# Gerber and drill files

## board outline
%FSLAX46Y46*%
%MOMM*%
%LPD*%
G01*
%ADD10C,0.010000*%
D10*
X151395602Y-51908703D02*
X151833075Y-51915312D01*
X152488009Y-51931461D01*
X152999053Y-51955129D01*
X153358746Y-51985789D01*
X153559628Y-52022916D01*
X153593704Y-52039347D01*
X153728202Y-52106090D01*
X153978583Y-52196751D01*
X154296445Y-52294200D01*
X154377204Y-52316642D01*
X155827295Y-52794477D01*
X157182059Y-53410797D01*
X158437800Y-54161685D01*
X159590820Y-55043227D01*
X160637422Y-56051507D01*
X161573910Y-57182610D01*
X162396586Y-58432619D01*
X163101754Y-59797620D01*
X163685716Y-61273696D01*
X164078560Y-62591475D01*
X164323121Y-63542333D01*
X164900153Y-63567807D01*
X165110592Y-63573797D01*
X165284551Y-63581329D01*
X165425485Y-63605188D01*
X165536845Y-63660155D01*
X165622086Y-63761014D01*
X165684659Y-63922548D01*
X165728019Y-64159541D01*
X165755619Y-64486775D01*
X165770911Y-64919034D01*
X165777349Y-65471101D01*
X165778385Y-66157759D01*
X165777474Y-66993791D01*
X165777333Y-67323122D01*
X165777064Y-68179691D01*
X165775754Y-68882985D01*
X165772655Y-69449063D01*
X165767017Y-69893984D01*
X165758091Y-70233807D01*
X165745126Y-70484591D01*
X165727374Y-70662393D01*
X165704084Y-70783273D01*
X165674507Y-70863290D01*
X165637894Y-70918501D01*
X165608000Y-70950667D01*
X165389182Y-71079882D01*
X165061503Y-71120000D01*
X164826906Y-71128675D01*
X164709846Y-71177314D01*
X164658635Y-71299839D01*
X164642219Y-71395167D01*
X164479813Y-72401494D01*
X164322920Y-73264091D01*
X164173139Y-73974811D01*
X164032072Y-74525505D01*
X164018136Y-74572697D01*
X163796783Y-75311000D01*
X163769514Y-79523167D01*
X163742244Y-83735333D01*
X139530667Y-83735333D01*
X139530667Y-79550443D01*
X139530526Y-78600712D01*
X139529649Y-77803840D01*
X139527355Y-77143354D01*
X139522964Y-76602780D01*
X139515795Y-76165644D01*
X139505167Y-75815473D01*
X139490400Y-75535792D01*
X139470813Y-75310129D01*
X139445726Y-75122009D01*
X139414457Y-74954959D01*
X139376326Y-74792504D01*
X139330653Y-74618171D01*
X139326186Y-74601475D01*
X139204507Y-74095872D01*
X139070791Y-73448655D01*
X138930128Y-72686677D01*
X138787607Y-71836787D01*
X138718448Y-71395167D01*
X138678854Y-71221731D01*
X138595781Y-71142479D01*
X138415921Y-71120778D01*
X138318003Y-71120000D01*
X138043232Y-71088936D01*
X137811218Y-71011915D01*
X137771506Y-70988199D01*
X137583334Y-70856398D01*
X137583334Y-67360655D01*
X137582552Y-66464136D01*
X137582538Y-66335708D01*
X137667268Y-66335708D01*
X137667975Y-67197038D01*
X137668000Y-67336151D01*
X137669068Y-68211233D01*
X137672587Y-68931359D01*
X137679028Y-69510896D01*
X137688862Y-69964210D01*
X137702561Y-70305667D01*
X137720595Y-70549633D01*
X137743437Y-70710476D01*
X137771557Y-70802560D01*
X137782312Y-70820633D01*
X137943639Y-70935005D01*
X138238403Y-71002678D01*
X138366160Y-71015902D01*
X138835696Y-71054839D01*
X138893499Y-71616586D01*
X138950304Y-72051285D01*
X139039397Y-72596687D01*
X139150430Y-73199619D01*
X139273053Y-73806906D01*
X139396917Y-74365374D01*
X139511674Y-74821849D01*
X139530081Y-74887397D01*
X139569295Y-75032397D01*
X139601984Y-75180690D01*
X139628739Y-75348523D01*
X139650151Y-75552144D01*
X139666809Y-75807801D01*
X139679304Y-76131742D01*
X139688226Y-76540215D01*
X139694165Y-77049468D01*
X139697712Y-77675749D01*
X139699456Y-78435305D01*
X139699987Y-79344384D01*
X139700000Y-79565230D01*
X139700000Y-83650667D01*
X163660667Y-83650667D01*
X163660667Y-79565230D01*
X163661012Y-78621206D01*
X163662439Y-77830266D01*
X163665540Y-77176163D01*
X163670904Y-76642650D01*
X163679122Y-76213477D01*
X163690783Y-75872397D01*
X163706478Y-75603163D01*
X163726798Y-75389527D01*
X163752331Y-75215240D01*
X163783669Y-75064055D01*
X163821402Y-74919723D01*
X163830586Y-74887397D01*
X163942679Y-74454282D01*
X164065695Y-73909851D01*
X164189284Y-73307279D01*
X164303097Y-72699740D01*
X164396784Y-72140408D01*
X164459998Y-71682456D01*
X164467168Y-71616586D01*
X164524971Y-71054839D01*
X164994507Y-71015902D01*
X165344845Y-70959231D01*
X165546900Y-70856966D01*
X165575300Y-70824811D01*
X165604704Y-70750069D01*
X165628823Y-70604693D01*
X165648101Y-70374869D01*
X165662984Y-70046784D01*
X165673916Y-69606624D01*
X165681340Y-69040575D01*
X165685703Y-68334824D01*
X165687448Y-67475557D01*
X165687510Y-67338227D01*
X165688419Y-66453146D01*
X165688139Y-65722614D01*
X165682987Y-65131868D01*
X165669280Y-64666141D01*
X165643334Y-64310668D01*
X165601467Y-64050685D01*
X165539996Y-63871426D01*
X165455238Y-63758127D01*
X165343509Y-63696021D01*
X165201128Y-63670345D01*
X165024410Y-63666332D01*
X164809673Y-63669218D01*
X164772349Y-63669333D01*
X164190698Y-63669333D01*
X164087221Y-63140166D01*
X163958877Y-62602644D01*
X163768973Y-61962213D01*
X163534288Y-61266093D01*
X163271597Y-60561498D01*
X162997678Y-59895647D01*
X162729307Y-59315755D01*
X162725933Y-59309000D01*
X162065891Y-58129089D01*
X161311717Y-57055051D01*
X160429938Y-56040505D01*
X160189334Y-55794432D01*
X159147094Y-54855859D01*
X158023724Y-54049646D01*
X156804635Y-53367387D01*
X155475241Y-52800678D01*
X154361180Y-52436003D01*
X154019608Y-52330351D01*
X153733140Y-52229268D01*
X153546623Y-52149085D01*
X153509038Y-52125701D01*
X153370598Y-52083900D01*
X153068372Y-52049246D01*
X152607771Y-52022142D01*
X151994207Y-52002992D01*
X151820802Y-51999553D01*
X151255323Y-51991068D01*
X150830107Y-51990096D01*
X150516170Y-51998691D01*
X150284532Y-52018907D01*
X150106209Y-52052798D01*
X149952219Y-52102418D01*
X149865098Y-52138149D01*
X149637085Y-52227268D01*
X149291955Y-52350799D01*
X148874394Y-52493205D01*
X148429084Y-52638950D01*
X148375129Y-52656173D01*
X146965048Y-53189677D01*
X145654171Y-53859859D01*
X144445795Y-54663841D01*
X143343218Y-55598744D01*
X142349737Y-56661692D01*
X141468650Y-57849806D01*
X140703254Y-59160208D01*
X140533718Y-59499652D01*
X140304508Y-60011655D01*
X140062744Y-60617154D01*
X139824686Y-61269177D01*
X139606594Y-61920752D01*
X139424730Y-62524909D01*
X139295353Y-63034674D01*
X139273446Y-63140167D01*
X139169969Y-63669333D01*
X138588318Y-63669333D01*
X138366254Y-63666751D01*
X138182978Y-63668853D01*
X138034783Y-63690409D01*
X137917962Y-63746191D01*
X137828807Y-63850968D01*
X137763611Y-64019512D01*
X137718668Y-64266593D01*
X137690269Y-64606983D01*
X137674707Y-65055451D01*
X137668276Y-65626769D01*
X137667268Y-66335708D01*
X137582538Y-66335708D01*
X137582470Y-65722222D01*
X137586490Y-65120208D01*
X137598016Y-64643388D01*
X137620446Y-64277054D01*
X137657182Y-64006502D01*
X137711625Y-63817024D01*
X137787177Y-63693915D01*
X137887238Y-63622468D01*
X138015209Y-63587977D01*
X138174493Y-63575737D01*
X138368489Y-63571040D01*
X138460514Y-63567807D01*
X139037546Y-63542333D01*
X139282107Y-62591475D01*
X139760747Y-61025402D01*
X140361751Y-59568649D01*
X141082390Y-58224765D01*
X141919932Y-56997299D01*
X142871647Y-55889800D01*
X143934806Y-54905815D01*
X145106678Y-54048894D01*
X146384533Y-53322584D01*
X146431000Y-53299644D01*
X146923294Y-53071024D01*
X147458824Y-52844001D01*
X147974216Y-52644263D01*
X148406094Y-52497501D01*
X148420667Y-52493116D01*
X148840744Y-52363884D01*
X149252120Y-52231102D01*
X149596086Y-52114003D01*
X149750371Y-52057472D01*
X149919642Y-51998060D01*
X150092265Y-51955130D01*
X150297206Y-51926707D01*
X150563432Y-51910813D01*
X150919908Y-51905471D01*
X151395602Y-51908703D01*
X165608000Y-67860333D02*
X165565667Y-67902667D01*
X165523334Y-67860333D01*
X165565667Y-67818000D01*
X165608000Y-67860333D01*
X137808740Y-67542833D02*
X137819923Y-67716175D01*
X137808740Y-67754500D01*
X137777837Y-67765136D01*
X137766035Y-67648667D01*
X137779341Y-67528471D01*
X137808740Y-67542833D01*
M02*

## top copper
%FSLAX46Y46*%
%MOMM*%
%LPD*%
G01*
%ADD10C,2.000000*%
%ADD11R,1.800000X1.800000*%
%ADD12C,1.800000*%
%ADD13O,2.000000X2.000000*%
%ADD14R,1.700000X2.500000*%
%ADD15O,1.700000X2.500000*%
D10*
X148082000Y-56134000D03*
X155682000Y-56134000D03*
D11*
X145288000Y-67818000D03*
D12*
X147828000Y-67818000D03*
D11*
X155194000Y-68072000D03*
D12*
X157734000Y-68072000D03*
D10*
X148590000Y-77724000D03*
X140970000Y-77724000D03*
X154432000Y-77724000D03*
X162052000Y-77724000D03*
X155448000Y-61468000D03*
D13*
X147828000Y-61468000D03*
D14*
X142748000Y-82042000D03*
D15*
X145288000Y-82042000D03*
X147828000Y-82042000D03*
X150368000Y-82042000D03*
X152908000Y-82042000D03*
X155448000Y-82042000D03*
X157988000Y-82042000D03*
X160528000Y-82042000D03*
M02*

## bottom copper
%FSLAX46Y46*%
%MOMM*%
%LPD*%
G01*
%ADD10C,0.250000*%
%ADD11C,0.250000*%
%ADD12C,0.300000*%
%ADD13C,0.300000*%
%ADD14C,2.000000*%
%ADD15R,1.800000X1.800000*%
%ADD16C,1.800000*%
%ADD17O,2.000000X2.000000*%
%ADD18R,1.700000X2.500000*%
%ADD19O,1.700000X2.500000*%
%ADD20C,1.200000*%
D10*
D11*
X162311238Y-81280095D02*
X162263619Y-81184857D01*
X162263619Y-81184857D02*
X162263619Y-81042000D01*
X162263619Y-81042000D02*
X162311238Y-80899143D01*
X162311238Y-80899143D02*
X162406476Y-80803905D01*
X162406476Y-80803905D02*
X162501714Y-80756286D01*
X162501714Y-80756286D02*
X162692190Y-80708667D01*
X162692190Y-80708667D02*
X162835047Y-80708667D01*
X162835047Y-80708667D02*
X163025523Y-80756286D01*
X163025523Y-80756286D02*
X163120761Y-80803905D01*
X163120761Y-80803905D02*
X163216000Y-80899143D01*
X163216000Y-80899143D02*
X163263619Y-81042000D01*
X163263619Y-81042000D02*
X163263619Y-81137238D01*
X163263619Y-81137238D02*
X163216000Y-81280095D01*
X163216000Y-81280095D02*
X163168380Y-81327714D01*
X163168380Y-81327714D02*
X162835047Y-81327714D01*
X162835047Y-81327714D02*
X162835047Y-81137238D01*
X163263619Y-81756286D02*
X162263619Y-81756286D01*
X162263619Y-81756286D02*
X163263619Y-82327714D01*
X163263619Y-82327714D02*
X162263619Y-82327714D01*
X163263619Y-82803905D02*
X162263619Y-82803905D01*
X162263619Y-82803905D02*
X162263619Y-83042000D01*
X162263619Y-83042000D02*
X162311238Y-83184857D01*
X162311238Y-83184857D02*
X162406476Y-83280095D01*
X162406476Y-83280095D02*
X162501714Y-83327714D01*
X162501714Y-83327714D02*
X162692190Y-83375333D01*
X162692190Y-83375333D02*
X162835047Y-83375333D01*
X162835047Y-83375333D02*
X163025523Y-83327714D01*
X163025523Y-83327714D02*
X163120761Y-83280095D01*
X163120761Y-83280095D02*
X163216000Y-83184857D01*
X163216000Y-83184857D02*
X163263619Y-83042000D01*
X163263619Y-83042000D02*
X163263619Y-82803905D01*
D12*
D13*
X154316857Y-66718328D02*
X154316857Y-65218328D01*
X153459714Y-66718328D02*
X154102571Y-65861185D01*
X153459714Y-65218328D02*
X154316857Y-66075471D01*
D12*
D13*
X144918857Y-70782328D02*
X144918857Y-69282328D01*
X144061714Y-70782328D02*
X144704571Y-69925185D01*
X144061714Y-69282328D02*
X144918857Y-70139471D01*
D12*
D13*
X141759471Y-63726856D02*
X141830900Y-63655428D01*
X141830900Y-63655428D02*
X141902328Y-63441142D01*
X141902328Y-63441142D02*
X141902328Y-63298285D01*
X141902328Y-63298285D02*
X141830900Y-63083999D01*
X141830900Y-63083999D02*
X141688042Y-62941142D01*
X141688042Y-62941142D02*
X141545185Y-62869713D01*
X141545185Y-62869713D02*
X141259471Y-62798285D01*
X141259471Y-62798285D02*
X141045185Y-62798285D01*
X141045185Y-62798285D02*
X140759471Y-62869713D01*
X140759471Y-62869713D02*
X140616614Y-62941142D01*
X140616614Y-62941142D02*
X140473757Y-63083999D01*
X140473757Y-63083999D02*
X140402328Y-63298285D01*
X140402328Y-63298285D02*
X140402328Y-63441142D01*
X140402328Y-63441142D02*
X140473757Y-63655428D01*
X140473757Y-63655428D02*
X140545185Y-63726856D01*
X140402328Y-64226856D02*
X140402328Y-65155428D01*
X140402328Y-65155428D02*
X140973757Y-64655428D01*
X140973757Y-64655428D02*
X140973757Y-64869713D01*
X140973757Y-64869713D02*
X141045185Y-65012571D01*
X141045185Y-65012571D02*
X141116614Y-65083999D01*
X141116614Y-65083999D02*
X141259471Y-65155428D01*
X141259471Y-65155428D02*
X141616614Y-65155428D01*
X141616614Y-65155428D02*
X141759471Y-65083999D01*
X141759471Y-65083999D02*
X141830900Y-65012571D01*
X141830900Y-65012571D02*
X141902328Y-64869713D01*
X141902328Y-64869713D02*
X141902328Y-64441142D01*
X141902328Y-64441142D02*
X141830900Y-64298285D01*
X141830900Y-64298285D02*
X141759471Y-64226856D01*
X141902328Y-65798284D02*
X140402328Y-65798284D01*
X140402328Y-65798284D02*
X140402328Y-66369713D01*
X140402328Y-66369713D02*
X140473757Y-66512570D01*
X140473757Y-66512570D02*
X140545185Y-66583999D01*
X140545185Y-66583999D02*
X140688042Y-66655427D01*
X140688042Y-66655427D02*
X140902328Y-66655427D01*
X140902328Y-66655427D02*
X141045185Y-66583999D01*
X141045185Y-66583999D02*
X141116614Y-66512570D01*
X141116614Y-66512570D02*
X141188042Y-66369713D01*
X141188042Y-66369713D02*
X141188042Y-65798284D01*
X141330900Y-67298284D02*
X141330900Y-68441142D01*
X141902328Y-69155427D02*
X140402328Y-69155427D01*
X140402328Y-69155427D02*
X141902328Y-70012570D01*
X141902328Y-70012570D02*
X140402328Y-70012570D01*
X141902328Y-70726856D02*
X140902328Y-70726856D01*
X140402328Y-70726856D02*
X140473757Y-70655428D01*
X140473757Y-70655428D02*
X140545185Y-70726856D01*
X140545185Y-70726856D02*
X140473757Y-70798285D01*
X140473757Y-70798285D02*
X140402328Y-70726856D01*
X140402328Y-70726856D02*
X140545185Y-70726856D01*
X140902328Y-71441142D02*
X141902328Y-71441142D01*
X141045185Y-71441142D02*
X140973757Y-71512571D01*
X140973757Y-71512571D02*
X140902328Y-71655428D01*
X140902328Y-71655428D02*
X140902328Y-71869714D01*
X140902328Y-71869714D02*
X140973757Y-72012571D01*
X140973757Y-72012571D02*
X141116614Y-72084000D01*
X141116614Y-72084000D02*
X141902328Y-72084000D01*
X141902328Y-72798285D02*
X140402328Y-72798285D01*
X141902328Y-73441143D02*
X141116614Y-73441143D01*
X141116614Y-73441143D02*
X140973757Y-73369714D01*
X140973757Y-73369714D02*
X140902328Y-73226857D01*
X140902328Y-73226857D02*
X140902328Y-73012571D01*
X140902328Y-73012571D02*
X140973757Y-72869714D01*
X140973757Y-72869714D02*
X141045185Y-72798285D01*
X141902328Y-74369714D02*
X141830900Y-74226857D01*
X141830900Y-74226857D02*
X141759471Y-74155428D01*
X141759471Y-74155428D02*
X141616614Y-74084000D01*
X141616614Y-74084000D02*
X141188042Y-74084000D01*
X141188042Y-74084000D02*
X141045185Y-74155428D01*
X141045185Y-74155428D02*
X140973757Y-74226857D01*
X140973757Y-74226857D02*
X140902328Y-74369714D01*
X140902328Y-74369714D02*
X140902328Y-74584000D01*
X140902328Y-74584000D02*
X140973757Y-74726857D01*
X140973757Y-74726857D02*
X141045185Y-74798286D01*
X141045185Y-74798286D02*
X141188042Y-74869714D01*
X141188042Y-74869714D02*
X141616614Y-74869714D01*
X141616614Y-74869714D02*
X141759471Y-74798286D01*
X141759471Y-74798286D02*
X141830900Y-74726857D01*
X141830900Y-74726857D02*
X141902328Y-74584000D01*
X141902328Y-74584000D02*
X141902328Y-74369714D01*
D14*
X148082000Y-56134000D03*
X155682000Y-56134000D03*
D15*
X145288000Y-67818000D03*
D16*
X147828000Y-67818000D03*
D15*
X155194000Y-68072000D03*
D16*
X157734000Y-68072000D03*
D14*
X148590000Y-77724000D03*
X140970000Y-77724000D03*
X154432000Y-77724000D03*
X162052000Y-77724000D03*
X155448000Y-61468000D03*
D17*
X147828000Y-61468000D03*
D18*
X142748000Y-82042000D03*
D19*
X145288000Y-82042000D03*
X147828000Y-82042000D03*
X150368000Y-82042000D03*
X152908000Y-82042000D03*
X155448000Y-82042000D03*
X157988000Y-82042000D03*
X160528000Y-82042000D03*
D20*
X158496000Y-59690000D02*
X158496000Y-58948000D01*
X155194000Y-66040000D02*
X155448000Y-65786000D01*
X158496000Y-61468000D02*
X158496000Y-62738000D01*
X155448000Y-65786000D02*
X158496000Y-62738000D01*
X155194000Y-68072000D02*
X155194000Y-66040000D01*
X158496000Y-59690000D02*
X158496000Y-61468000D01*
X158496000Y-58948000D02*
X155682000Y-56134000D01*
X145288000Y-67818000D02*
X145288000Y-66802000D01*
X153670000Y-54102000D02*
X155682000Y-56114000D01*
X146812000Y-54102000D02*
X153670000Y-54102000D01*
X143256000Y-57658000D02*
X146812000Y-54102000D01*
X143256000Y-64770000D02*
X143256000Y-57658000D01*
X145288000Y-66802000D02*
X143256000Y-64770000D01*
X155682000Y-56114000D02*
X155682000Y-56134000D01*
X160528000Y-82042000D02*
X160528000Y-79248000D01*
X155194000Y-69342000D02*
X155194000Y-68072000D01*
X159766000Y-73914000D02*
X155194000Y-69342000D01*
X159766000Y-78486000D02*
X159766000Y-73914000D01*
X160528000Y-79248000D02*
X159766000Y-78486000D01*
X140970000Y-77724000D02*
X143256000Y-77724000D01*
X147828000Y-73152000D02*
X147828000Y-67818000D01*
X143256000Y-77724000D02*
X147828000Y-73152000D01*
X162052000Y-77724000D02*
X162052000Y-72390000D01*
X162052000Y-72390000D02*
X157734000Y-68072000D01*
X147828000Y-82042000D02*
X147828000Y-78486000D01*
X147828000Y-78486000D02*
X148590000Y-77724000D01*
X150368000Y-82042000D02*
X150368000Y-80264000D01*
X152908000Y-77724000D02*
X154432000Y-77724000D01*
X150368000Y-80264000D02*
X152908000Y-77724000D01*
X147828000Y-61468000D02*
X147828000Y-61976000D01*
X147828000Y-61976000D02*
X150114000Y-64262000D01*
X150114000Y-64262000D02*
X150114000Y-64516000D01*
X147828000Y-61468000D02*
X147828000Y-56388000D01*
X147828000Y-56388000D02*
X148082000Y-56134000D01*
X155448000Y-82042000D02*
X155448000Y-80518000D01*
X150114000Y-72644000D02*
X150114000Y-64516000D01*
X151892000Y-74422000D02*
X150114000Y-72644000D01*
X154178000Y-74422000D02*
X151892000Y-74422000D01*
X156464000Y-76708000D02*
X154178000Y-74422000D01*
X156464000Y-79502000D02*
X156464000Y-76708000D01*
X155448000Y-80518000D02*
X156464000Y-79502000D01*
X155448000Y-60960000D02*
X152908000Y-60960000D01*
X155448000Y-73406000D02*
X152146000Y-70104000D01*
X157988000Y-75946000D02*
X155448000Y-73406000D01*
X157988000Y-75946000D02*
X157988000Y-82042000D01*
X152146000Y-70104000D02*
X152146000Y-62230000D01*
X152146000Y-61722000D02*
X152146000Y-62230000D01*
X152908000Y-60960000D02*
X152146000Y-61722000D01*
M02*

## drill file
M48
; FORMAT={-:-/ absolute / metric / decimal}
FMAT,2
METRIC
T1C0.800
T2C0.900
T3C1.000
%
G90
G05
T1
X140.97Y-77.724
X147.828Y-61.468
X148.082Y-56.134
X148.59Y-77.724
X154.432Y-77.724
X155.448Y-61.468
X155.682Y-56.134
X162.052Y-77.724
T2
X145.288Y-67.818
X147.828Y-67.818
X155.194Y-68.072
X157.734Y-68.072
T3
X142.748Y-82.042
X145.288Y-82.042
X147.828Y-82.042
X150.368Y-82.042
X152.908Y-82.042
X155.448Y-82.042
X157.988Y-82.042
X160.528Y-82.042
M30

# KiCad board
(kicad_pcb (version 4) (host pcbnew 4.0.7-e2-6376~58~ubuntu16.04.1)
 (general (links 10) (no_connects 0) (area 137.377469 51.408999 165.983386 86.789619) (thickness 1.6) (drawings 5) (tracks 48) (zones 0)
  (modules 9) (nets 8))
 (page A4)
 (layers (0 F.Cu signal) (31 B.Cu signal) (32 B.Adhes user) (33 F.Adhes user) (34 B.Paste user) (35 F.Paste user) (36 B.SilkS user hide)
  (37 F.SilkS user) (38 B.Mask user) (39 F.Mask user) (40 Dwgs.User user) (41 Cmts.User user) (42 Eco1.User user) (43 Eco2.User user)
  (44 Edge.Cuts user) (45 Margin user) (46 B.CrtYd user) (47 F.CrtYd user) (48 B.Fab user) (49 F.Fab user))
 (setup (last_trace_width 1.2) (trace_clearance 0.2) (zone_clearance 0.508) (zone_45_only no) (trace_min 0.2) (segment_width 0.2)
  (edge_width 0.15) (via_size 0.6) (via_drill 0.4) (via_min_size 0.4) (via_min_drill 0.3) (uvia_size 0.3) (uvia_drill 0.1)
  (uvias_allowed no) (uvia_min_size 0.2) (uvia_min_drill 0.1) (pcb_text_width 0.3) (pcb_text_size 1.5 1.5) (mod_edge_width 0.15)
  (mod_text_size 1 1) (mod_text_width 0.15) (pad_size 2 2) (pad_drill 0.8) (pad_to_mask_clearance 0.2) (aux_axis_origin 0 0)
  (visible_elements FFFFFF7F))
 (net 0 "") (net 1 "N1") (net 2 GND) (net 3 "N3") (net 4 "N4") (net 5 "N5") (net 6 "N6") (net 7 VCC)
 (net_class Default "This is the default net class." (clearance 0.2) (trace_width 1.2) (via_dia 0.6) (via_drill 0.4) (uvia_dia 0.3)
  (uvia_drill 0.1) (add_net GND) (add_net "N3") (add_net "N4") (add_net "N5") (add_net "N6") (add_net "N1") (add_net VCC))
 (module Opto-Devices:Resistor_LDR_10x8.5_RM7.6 (layer F.Cu) (at 148.082 56.134)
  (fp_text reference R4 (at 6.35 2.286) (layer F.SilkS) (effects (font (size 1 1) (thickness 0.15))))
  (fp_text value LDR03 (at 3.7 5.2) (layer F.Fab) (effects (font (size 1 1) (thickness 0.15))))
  (pad 1 thru_hole circle (at 0 0) (size 2 2) (drill 0.8) (layers *.Cu *.Mask) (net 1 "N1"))
  (pad 2 thru_hole circle (at 7.6 0) (size 2 2) (drill 0.8) (layers *.Cu *.Mask) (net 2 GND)))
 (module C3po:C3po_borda (layer F.Cu) (at 151.638 67.818)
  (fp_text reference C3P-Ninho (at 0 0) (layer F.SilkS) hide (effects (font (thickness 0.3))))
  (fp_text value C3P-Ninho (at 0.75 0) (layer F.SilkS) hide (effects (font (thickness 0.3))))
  (fp_poly
   (pts (xy -0.242398 -15.909297) (xy 0.195075 -15.902688) (xy 0.850009 -15.886539) (xy 1.361053 -15.862871) (xy 1.720746 -15.832211)
    (xy 1.921628 -15.795084) (xy 1.955704 -15.778653) (xy 2.090202 -15.71191) (xy 2.340583 -15.621249) (xy 2.658445 -15.5238)
    (xy 2.739204 -15.501358) (xy 4.189295 -15.023523) (xy 5.544059 -14.407203) (xy 6.7998 -13.656315) (xy 7.95282 -12.774773)
    (xy 8.999422 -11.766493) (xy 9.93591 -10.63539) (xy 10.758586 -9.385381) (xy 11.463754 -8.02038) (xy 12.047716 -6.544304)
    (xy 12.44056 -5.226525) (xy 12.685121 -4.275667) (xy 13.262153 -4.250193) (xy 13.472592 -4.244203) (xy 13.646551 -4.236671)
    (xy 13.787485 -4.212812) (xy 13.898845 -4.157845) (xy 13.984086 -4.056986) (xy 14.046659 -3.895452) (xy 14.090019 -3.658459)
    (xy 14.117619 -3.331225) (xy 14.132911 -2.898966) (xy 14.139349 -2.346899) (xy 14.140385 -1.660241) (xy 14.139474 -0.824209)
    (xy 14.139333 -0.494878) (xy 14.139064 0.361691) (xy 14.137754 1.064985) (xy 14.134655 1.631063) (xy 14.129017 2.075984)
    (xy 14.120091 2.415807) (xy 14.107126 2.666591) (xy 14.089374 2.844393) (xy 14.066084 2.965273) (xy 14.036507 3.04529)
    (xy 13.999894 3.100501) (xy 13.97 3.132667) (xy 13.751182 3.261882) (xy 13.423503 3.302) (xy 13.188906 3.310675) (xy 13.071846 3.359314)
    (xy 13.020635 3.481839) (xy 13.004219 3.577167) (xy 12.841813 4.583494) (xy 12.68492 5.446091) (xy 12.535139 6.156811)
    (xy 12.394072 6.707505) (xy 12.380136 6.754697) (xy 12.158783 7.493) (xy 12.131514 11.705167) (xy 12.104244 15.917333)
    (xy -12.107333 15.917333) (xy -12.107333 11.732443) (xy -12.107474 10.782712) (xy -12.108351 9.98584) (xy -12.110645 9.325354)
    (xy -12.115036 8.78478) (xy -12.122205 8.347644) (xy -12.132833 7.997473) (xy -12.1476 7.717792) (xy -12.167187 7.492129)
    (xy -12.192274 7.304009) (xy -12.223543 7.136959) (xy -12.261674 6.974504) (xy -12.307347 6.800171) (xy -12.311814 6.783475)
    (xy -12.433493 6.277872) (xy -12.567209 5.630655) (xy -12.707872 4.868677) (xy -12.850393 4.018787) (xy -12.919552 3.577167)
    (xy -12.959146 3.403731) (xy -13.042219 3.324479) (xy -13.222079 3.302778) (xy -13.319997 3.302) (xy -13.594768 3.270936)
    (xy -13.826782 3.193915) (xy -13.866494 3.170199) (xy -14.054666 3.038398) (xy -14.054666 -0.457345) (xy -14.055448 -1.353864)
    (xy -14.055462 -1.482292) (xy -13.970732 -1.482292) (xy -13.970025 -0.620962) (xy -13.97 -0.481849) (xy -13.968932 0.393233)
    (xy -13.965413 1.113359) (xy -13.958972 1.692896) (xy -13.949138 2.14621) (xy -13.935439 2.487667) (xy -13.917405 2.731633)
    (xy -13.894563 2.892476) (xy -13.866443 2.98456) (xy -13.855688 3.002633) (xy -13.694361 3.117005) (xy -13.399597 3.184678)
    (xy -13.27184 3.197902) (xy -12.802304 3.236839) (xy -12.744501 3.798586) (xy -12.687696 4.233285) (xy -12.598603 4.778687)
    (xy -12.48757 5.381619) (xy -12.364947 5.988906) (xy -12.241083 6.547374) (xy -12.126326 7.003849) (xy -12.107919 7.069397)
    (xy -12.068705 7.214397) (xy -12.036016 7.36269) (xy -12.009261 7.530523) (xy -11.987849 7.734144) (xy -11.971191 7.989801)
    (xy -11.958696 8.313742) (xy -11.949774 8.722215) (xy -11.943835 9.231468) (xy -11.940288 9.857749) (xy -11.938544 10.617305)
    (xy -11.938013 11.526384) (xy -11.938 11.74723) (xy -11.938 15.832667) (xy 12.022667 15.832667) (xy 12.022667 11.74723)
    (xy 12.023012 10.803206) (xy 12.024439 10.012266) (xy 12.02754 9.358163) (xy 12.032904 8.82465) (xy 12.041122 8.395477)
    (xy 12.052783 8.054397) (xy 12.068478 7.785163) (xy 12.088798 7.571527) (xy 12.114331 7.39724) (xy 12.145669 7.246055)
    (xy 12.183402 7.101723) (xy 12.192586 7.069397) (xy 12.304679 6.636282) (xy 12.427695 6.091851) (xy 12.551284 5.489279)
    (xy 12.665097 4.88174) (xy 12.758784 4.322408) (xy 12.821998 3.864456) (xy 12.829168 3.798586) (xy 12.886971 3.236839)
    (xy 13.356507 3.197902) (xy 13.706845 3.141231) (xy 13.9089 3.038966) (xy 13.9373 3.006811) (xy 13.966704 2.932069)
    (xy 13.990823 2.786693) (xy 14.010101 2.556869) (xy 14.024984 2.228784) (xy 14.035916 1.788624) (xy 14.04334 1.222575)
    (xy 14.047703 0.516824) (xy 14.049448 -0.342443) (xy 14.04951 -0.479773) (xy 14.050419 -1.364854) (xy 14.050139 -2.095386)
    (xy 14.044987 -2.686132) (xy 14.03128 -3.151859) (xy 14.005334 -3.507332) (xy 13.963467 -3.767315) (xy 13.901996 -3.946574)
    (xy 13.817238 -4.059873) (xy 13.705509 -4.121979) (xy 13.563128 -4.147655) (xy 13.38641 -4.151668) (xy 13.171673 -4.148782)
    (xy 13.134349 -4.148667) (xy 12.552698 -4.148667) (xy 12.449221 -4.677834) (xy 12.320877 -5.215356) (xy 12.130973 -5.855787)
    (xy 11.896288 -6.551907) (xy 11.633597 -7.256502) (xy 11.359678 -7.922353) (xy 11.091307 -8.502245) (xy 11.087933 -8.509)
    (xy 10.427891 -9.688911) (xy 9.673717 -10.762949) (xy 8.791938 -11.777495) (xy 8.551334 -12.023568) (xy 7.509094 -12.962141)
    (xy 6.385724 -13.768354) (xy 5.166635 -14.450613) (xy 3.837241 -15.017322) (xy 2.72318 -15.381997) (xy 2.381608 -15.487649)
    (xy 2.09514 -15.588732) (xy 1.908623 -15.668915) (xy 1.871038 -15.692299) (xy 1.732598 -15.7341) (xy 1.430372 -15.768754)
    (xy 0.969771 -15.795858) (xy 0.356207 -15.815008) (xy 0.182802 -15.818447) (xy -0.382677 -15.826932) (xy -0.807893 -15.827904)
    (xy -1.12183 -15.819309) (xy -1.353468 -15.799093) (xy -1.531791 -15.765202) (xy -1.685781 -15.715582) (xy -1.772902 -15.679851)
    (xy -2.000915 -15.590732) (xy -2.346045 -15.467201) (xy -2.763606 -15.324795) (xy -3.208916 -15.17905) (xy -3.262871 -15.161827)
    (xy -4.672952 -14.628323) (xy -5.983829 -13.958141) (xy -7.192205 -13.154159) (xy -8.294782 -12.219256) (xy -9.288263 -11.156308)
    (xy -10.16935 -9.968194) (xy -10.934746 -8.657792) (xy -11.104282 -8.318348) (xy -11.333492 -7.806345) (xy -11.575256 -7.200846)
    (xy -11.813314 -6.548823) (xy -12.031406 -5.897248) (xy -12.21327 -5.293091) (xy -12.342647 -4.783326) (xy -12.364554 -4.677833)
    (xy -12.468031 -4.148667) (xy -13.049682 -4.148667) (xy -13.271746 -4.151249) (xy -13.455022 -4.149147) (xy -13.603217 -4.127591)
    (xy -13.720038 -4.071809) (xy -13.809193 -3.967032) (xy -13.874389 -3.798488) (xy -13.919332 -3.551407) (xy -13.947731 -3.211017)
    (xy -13.963293 -2.762549) (xy -13.969724 -2.191231) (xy -13.970732 -1.482292) (xy -14.055462 -1.482292) (xy -14.05553 -2.095778)
    (xy -14.05151 -2.697792) (xy -14.039984 -3.174612) (xy -14.017554 -3.540946) (xy -13.980818 -3.811498) (xy -13.926375 -4.000976)
    (xy -13.850823 -4.124085) (xy -13.750762 -4.195532) (xy -13.622791 -4.230023) (xy -13.463507 -4.242263) (xy -13.269511 -4.24696)
    (xy -13.177486 -4.250193) (xy -12.600454 -4.275667) (xy -12.355893 -5.226525) (xy -11.877253 -6.792598) (xy -11.276249 -8.249351)
    (xy -10.55561 -9.593235) (xy -9.718068 -10.820701) (xy -8.766353 -11.9282) (xy -7.703194 -12.912185) (xy -6.531322 -13.769106)
    (xy -5.253467 -14.495416) (xy -5.207 -14.518356) (xy -4.714706 -14.746976) (xy -4.179176 -14.973999) (xy -3.663784 -15.173737)
    (xy -3.231906 -15.320499) (xy -3.217333 -15.324884) (xy -2.797256 -15.454116) (xy -2.38588 -15.586898) (xy -2.041914 -15.703997)
    (xy -1.887629 -15.760528) (xy -1.718358 -15.81994) (xy -1.545735 -15.86287) (xy -1.340794 -15.891293) (xy -1.074568 -15.907187)
    (xy -0.718092 -15.912529) (xy -0.242398 -15.909297))
   (layer Edge.Cuts) (width 0.01))
  (fp_poly
   (pts (xy 13.97 0.042333) (xy 13.927667 0.084667) (xy 13.885334 0.042333) (xy 13.927667 0) (xy 13.97 0.042333)) (layer Edge.Cuts)
   (width 0.01))
  (fp_poly
   (pts (xy -13.82926 -0.275167) (xy -13.818077 -0.101825) (xy -13.82926 -0.0635) (xy -13.860163 -0.052864) (xy -13.871965 -0.169333)
    (xy -13.858659 -0.289529) (xy -13.82926 -0.275167))
   (layer Edge.Cuts) (width 0.01)))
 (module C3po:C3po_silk (layer F.Cu) (at 151.638 66.802)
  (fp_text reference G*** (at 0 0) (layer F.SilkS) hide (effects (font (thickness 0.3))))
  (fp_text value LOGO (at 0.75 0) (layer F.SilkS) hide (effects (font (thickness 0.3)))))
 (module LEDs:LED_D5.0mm (layer F.Cu) (at 145.288 67.818)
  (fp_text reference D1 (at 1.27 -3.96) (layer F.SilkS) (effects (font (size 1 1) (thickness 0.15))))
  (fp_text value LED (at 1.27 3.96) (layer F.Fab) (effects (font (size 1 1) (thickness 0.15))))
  (pad 1 thru_hole rect (at 0 0) (size 1.8 1.8) (drill 0.9) (layers *.Cu *.Mask) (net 2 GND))
  (pad 2 thru_hole circle (at 2.54 0) (size 1.8 1.8) (drill 0.9) (layers *.Cu *.Mask) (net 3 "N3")))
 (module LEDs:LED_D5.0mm (layer F.Cu) (at 155.194 68.072)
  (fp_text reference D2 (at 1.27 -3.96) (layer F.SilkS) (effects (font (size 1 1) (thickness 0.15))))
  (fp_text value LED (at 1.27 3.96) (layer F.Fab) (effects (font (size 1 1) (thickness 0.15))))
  (pad 1 thru_hole rect (at 0 0) (size 1.8 1.8) (drill 0.9) (layers *.Cu *.Mask) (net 2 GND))
  (pad 2 thru_hole circle (at 2.54 0) (size 1.8 1.8) (drill 0.9) (layers *.Cu *.Mask) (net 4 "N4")))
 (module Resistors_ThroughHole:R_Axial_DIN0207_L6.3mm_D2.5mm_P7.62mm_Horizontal (layer F.Cu) (at 148.59 77.724 180)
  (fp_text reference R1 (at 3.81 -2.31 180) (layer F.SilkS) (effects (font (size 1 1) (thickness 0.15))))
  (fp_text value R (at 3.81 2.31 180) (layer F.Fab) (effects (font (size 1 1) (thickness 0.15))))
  (pad 1 thru_hole circle (at 0 0 180) (size 2 2) (drill 0.8) (layers *.Cu *.Mask) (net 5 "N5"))
  (pad 2 thru_hole circle (at 7.62 0 180) (size 2 2) (drill 0.8) (layers *.Cu *.Mask) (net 3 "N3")))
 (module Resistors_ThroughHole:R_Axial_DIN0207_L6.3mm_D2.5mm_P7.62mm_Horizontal (layer F.Cu) (at 154.432 77.724)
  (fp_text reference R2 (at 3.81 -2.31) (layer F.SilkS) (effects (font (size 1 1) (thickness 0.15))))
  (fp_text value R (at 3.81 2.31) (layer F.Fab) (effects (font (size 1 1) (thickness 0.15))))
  (pad 1 thru_hole circle (at 0 0) (size 2 2) (drill 0.8) (layers *.Cu *.Mask) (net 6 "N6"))
  (pad 2 thru_hole circle (at 7.62 0) (size 2 2) (drill 0.8) (layers *.Cu *.Mask) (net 4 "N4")))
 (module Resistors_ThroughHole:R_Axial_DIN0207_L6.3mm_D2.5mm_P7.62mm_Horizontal (layer F.Cu) (at 155.448 61.468 180)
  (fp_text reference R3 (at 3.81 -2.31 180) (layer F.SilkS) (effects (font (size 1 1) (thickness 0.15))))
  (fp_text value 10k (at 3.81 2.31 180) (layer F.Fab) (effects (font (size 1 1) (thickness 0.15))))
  (pad 1 thru_hole circle (at 0 0 180) (size 2 2) (drill 0.8) (layers *.Cu *.Mask) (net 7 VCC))
  (pad 2 thru_hole oval (at 7.62 0 180) (size 2 2) (drill 0.8) (layers *.Cu *.Mask) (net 1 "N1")))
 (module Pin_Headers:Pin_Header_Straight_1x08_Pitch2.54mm (layer F.Cu) (at 142.748 82.042 90)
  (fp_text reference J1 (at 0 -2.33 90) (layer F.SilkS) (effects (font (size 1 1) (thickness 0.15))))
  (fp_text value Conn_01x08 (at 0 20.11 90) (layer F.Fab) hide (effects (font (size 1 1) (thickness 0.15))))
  (pad 1 thru_hole rect (at 0 0 90) (size 2.5 1.7) (drill 1) (layers *.Cu *.Mask))
  (pad 2 thru_hole oval (at 0 2.54 90) (size 2.5 1.7) (drill 1) (layers *.Cu *.Mask))
  (pad 3 thru_hole oval (at 0 5.08 90) (size 2.5 1.7) (drill 1) (layers *.Cu *.Mask) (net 5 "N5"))
  (pad 4 thru_hole oval (at 0 7.62 90) (size 2.5 1.7) (drill 1) (layers *.Cu *.Mask) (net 6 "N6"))
  (pad 5 thru_hole oval (at 0 10.16 90) (size 2.5 1.7) (drill 1) (layers *.Cu *.Mask))
  (pad 6 thru_hole oval (at 0 12.7 90) (size 2.5 1.7) (drill 1) (layers *.Cu *.Mask) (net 1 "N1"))
  (pad 7 thru_hole oval (at 0 15.24 90) (size 2.5 1.7) (drill 1) (layers *.Cu *.Mask) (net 7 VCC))
  (pad 8 thru_hole oval (at 0 17.78 90) (size 2.5 1.7) (drill 1) (layers *.Cu *.Mask) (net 2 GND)))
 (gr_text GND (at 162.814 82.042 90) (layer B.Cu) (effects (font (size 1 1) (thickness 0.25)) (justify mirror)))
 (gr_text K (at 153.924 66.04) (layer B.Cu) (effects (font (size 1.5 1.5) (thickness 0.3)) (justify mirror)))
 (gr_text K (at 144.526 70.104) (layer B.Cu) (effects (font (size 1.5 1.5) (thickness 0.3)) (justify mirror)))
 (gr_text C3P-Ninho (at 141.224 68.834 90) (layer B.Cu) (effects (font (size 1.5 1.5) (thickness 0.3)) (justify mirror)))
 (segment (start 158.496 59.69) (end 158.496 58.948) (width 1.2) (layer B.Cu) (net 2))
 (segment (start 155.194 66.04) (end 155.448 65.786) (width 1.2) (layer B.Cu) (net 2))
 (segment (start 158.496 61.468) (end 158.496 62.738) (width 1.2) (layer B.Cu) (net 2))
 (segment (start 155.448 65.786) (end 158.496 62.738) (width 1.2) (layer B.Cu) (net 2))
 (segment (start 155.194 68.072) (end 155.194 66.04) (width 1.2) (layer B.Cu) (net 2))
 (segment (start 158.496 59.69) (end 158.496 61.468) (width 1.2) (layer B.Cu) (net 2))
 (segment (start 158.496 58.948) (end 155.682 56.134) (width 1.2) (layer B.Cu) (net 2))
 (segment (start 145.288 67.818) (end 145.288 66.802) (width 1.2) (layer B.Cu) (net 2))
 (segment (start 153.67 54.102) (end 155.682 56.114) (width 1.2) (layer B.Cu) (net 2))
 (segment (start 146.812 54.102) (end 153.67 54.102) (width 1.2) (layer B.Cu) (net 2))
 (segment (start 143.256 57.658) (end 146.812 54.102) (width 1.2) (layer B.Cu) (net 2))
 (segment (start 143.256 64.77) (end 143.256 57.658) (width 1.2) (layer B.Cu) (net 2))
 (segment (start 145.288 66.802) (end 143.256 64.77) (width 1.2) (layer B.Cu) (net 2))
 (segment (start 155.682 56.114) (end 155.682 56.134) (width 1.2) (layer B.Cu) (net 2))
 (segment (start 160.528 82.042) (end 160.528 79.248) (width 1.2) (layer B.Cu) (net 2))
 (segment (start 155.194 69.342) (end 155.194 68.072) (width 1.2) (layer B.Cu) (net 2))
 (segment (start 159.766 73.914) (end 155.194 69.342) (width 1.2) (layer B.Cu) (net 2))
 (segment (start 159.766 78.486) (end 159.766 73.914) (width 1.2) (layer B.Cu) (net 2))
 (segment (start 160.528 79.248) (end 159.766 78.486) (width 1.2) (layer B.Cu) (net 2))
 (segment (start 140.97 77.724) (end 143.256 77.724) (width 1.2) (layer B.Cu) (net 3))
 (segment (start 147.828 73.152) (end 147.828 67.818) (width 1.2) (layer B.Cu) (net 3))
 (segment (start 143.256 77.724) (end 147.828 73.152) (width 1.2) (layer B.Cu) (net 3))
 (segment (start 162.052 77.724) (end 162.052 72.39) (width 1.2) (layer B.Cu) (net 4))
 (segment (start 162.052 72.39) (end 157.734 68.072) (width 1.2) (layer B.Cu) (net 4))
 (segment (start 147.828 82.042) (end 147.828 78.486) (width 1.2) (layer B.Cu) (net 5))
 (segment (start 147.828 78.486) (end 148.59 77.724) (width 1.2) (layer B.Cu) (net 5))
 (segment (start 150.368 82.042) (end 150.368 80.264) (width 1.2) (layer B.Cu) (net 6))
 (segment (start 152.908 77.724) (end 154.432 77.724) (width 1.2) (layer B.Cu) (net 6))
 (segment (start 150.368 80.264) (end 152.908 77.724) (width 1.2) (layer B.Cu) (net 6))
 (segment (start 147.828 61.468) (end 147.828 61.976) (width 1.2) (layer B.Cu) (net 1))
 (segment (start 147.828 61.976) (end 150.114 64.262) (width 1.2) (layer B.Cu) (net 1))
 (segment (start 150.114 64.262) (end 150.114 64.516) (width 1.2) (layer B.Cu) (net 1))
 (segment (start 147.828 61.468) (end 147.828 56.388) (width 1.2) (layer B.Cu) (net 1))
 (segment (start 147.828 56.388) (end 148.082 56.134) (width 1.2) (layer B.Cu) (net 1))
 (segment (start 155.448 82.042) (end 155.448 80.518) (width 1.2) (layer B.Cu) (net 1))
 (segment (start 150.114 72.644) (end 150.114 64.516) (width 1.2) (layer B.Cu) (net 1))
 (segment (start 151.892 74.422) (end 150.114 72.644) (width 1.2) (layer B.Cu) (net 1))
 (segment (start 154.178 74.422) (end 151.892 74.422) (width 1.2) (layer B.Cu) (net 1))
 (segment (start 156.464 76.708) (end 154.178 74.422) (width 1.2) (layer B.Cu) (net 1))
 (segment (start 156.464 79.502) (end 156.464 76.708) (width 1.2) (layer B.Cu) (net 1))
 (segment (start 155.448 80.518) (end 156.464 79.502) (width 1.2) (layer B.Cu) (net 1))
 (segment (start 155.448 60.96) (end 152.908 60.96) (width 1.2) (layer B.Cu) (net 7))
 (segment (start 155.448 73.406) (end 152.146 70.104) (width 1.2) (layer B.Cu) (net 7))
 (segment (start 157.988 75.946) (end 155.448 73.406) (width 1.2) (layer B.Cu) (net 7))
 (segment (start 157.988 75.946) (end 157.988 82.042) (width 1.2) (layer B.Cu) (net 7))
 (segment (start 152.146 70.104) (end 152.146 62.23) (width 1.2) (layer B.Cu) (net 7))
 (segment (start 152.146 61.722) (end 152.146 62.23) (width 1.2) (layer B.Cu) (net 7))
 (segment (start 152.908 60.96) (end 152.146 61.722) (width 1.2) (layer B.Cu) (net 7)))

